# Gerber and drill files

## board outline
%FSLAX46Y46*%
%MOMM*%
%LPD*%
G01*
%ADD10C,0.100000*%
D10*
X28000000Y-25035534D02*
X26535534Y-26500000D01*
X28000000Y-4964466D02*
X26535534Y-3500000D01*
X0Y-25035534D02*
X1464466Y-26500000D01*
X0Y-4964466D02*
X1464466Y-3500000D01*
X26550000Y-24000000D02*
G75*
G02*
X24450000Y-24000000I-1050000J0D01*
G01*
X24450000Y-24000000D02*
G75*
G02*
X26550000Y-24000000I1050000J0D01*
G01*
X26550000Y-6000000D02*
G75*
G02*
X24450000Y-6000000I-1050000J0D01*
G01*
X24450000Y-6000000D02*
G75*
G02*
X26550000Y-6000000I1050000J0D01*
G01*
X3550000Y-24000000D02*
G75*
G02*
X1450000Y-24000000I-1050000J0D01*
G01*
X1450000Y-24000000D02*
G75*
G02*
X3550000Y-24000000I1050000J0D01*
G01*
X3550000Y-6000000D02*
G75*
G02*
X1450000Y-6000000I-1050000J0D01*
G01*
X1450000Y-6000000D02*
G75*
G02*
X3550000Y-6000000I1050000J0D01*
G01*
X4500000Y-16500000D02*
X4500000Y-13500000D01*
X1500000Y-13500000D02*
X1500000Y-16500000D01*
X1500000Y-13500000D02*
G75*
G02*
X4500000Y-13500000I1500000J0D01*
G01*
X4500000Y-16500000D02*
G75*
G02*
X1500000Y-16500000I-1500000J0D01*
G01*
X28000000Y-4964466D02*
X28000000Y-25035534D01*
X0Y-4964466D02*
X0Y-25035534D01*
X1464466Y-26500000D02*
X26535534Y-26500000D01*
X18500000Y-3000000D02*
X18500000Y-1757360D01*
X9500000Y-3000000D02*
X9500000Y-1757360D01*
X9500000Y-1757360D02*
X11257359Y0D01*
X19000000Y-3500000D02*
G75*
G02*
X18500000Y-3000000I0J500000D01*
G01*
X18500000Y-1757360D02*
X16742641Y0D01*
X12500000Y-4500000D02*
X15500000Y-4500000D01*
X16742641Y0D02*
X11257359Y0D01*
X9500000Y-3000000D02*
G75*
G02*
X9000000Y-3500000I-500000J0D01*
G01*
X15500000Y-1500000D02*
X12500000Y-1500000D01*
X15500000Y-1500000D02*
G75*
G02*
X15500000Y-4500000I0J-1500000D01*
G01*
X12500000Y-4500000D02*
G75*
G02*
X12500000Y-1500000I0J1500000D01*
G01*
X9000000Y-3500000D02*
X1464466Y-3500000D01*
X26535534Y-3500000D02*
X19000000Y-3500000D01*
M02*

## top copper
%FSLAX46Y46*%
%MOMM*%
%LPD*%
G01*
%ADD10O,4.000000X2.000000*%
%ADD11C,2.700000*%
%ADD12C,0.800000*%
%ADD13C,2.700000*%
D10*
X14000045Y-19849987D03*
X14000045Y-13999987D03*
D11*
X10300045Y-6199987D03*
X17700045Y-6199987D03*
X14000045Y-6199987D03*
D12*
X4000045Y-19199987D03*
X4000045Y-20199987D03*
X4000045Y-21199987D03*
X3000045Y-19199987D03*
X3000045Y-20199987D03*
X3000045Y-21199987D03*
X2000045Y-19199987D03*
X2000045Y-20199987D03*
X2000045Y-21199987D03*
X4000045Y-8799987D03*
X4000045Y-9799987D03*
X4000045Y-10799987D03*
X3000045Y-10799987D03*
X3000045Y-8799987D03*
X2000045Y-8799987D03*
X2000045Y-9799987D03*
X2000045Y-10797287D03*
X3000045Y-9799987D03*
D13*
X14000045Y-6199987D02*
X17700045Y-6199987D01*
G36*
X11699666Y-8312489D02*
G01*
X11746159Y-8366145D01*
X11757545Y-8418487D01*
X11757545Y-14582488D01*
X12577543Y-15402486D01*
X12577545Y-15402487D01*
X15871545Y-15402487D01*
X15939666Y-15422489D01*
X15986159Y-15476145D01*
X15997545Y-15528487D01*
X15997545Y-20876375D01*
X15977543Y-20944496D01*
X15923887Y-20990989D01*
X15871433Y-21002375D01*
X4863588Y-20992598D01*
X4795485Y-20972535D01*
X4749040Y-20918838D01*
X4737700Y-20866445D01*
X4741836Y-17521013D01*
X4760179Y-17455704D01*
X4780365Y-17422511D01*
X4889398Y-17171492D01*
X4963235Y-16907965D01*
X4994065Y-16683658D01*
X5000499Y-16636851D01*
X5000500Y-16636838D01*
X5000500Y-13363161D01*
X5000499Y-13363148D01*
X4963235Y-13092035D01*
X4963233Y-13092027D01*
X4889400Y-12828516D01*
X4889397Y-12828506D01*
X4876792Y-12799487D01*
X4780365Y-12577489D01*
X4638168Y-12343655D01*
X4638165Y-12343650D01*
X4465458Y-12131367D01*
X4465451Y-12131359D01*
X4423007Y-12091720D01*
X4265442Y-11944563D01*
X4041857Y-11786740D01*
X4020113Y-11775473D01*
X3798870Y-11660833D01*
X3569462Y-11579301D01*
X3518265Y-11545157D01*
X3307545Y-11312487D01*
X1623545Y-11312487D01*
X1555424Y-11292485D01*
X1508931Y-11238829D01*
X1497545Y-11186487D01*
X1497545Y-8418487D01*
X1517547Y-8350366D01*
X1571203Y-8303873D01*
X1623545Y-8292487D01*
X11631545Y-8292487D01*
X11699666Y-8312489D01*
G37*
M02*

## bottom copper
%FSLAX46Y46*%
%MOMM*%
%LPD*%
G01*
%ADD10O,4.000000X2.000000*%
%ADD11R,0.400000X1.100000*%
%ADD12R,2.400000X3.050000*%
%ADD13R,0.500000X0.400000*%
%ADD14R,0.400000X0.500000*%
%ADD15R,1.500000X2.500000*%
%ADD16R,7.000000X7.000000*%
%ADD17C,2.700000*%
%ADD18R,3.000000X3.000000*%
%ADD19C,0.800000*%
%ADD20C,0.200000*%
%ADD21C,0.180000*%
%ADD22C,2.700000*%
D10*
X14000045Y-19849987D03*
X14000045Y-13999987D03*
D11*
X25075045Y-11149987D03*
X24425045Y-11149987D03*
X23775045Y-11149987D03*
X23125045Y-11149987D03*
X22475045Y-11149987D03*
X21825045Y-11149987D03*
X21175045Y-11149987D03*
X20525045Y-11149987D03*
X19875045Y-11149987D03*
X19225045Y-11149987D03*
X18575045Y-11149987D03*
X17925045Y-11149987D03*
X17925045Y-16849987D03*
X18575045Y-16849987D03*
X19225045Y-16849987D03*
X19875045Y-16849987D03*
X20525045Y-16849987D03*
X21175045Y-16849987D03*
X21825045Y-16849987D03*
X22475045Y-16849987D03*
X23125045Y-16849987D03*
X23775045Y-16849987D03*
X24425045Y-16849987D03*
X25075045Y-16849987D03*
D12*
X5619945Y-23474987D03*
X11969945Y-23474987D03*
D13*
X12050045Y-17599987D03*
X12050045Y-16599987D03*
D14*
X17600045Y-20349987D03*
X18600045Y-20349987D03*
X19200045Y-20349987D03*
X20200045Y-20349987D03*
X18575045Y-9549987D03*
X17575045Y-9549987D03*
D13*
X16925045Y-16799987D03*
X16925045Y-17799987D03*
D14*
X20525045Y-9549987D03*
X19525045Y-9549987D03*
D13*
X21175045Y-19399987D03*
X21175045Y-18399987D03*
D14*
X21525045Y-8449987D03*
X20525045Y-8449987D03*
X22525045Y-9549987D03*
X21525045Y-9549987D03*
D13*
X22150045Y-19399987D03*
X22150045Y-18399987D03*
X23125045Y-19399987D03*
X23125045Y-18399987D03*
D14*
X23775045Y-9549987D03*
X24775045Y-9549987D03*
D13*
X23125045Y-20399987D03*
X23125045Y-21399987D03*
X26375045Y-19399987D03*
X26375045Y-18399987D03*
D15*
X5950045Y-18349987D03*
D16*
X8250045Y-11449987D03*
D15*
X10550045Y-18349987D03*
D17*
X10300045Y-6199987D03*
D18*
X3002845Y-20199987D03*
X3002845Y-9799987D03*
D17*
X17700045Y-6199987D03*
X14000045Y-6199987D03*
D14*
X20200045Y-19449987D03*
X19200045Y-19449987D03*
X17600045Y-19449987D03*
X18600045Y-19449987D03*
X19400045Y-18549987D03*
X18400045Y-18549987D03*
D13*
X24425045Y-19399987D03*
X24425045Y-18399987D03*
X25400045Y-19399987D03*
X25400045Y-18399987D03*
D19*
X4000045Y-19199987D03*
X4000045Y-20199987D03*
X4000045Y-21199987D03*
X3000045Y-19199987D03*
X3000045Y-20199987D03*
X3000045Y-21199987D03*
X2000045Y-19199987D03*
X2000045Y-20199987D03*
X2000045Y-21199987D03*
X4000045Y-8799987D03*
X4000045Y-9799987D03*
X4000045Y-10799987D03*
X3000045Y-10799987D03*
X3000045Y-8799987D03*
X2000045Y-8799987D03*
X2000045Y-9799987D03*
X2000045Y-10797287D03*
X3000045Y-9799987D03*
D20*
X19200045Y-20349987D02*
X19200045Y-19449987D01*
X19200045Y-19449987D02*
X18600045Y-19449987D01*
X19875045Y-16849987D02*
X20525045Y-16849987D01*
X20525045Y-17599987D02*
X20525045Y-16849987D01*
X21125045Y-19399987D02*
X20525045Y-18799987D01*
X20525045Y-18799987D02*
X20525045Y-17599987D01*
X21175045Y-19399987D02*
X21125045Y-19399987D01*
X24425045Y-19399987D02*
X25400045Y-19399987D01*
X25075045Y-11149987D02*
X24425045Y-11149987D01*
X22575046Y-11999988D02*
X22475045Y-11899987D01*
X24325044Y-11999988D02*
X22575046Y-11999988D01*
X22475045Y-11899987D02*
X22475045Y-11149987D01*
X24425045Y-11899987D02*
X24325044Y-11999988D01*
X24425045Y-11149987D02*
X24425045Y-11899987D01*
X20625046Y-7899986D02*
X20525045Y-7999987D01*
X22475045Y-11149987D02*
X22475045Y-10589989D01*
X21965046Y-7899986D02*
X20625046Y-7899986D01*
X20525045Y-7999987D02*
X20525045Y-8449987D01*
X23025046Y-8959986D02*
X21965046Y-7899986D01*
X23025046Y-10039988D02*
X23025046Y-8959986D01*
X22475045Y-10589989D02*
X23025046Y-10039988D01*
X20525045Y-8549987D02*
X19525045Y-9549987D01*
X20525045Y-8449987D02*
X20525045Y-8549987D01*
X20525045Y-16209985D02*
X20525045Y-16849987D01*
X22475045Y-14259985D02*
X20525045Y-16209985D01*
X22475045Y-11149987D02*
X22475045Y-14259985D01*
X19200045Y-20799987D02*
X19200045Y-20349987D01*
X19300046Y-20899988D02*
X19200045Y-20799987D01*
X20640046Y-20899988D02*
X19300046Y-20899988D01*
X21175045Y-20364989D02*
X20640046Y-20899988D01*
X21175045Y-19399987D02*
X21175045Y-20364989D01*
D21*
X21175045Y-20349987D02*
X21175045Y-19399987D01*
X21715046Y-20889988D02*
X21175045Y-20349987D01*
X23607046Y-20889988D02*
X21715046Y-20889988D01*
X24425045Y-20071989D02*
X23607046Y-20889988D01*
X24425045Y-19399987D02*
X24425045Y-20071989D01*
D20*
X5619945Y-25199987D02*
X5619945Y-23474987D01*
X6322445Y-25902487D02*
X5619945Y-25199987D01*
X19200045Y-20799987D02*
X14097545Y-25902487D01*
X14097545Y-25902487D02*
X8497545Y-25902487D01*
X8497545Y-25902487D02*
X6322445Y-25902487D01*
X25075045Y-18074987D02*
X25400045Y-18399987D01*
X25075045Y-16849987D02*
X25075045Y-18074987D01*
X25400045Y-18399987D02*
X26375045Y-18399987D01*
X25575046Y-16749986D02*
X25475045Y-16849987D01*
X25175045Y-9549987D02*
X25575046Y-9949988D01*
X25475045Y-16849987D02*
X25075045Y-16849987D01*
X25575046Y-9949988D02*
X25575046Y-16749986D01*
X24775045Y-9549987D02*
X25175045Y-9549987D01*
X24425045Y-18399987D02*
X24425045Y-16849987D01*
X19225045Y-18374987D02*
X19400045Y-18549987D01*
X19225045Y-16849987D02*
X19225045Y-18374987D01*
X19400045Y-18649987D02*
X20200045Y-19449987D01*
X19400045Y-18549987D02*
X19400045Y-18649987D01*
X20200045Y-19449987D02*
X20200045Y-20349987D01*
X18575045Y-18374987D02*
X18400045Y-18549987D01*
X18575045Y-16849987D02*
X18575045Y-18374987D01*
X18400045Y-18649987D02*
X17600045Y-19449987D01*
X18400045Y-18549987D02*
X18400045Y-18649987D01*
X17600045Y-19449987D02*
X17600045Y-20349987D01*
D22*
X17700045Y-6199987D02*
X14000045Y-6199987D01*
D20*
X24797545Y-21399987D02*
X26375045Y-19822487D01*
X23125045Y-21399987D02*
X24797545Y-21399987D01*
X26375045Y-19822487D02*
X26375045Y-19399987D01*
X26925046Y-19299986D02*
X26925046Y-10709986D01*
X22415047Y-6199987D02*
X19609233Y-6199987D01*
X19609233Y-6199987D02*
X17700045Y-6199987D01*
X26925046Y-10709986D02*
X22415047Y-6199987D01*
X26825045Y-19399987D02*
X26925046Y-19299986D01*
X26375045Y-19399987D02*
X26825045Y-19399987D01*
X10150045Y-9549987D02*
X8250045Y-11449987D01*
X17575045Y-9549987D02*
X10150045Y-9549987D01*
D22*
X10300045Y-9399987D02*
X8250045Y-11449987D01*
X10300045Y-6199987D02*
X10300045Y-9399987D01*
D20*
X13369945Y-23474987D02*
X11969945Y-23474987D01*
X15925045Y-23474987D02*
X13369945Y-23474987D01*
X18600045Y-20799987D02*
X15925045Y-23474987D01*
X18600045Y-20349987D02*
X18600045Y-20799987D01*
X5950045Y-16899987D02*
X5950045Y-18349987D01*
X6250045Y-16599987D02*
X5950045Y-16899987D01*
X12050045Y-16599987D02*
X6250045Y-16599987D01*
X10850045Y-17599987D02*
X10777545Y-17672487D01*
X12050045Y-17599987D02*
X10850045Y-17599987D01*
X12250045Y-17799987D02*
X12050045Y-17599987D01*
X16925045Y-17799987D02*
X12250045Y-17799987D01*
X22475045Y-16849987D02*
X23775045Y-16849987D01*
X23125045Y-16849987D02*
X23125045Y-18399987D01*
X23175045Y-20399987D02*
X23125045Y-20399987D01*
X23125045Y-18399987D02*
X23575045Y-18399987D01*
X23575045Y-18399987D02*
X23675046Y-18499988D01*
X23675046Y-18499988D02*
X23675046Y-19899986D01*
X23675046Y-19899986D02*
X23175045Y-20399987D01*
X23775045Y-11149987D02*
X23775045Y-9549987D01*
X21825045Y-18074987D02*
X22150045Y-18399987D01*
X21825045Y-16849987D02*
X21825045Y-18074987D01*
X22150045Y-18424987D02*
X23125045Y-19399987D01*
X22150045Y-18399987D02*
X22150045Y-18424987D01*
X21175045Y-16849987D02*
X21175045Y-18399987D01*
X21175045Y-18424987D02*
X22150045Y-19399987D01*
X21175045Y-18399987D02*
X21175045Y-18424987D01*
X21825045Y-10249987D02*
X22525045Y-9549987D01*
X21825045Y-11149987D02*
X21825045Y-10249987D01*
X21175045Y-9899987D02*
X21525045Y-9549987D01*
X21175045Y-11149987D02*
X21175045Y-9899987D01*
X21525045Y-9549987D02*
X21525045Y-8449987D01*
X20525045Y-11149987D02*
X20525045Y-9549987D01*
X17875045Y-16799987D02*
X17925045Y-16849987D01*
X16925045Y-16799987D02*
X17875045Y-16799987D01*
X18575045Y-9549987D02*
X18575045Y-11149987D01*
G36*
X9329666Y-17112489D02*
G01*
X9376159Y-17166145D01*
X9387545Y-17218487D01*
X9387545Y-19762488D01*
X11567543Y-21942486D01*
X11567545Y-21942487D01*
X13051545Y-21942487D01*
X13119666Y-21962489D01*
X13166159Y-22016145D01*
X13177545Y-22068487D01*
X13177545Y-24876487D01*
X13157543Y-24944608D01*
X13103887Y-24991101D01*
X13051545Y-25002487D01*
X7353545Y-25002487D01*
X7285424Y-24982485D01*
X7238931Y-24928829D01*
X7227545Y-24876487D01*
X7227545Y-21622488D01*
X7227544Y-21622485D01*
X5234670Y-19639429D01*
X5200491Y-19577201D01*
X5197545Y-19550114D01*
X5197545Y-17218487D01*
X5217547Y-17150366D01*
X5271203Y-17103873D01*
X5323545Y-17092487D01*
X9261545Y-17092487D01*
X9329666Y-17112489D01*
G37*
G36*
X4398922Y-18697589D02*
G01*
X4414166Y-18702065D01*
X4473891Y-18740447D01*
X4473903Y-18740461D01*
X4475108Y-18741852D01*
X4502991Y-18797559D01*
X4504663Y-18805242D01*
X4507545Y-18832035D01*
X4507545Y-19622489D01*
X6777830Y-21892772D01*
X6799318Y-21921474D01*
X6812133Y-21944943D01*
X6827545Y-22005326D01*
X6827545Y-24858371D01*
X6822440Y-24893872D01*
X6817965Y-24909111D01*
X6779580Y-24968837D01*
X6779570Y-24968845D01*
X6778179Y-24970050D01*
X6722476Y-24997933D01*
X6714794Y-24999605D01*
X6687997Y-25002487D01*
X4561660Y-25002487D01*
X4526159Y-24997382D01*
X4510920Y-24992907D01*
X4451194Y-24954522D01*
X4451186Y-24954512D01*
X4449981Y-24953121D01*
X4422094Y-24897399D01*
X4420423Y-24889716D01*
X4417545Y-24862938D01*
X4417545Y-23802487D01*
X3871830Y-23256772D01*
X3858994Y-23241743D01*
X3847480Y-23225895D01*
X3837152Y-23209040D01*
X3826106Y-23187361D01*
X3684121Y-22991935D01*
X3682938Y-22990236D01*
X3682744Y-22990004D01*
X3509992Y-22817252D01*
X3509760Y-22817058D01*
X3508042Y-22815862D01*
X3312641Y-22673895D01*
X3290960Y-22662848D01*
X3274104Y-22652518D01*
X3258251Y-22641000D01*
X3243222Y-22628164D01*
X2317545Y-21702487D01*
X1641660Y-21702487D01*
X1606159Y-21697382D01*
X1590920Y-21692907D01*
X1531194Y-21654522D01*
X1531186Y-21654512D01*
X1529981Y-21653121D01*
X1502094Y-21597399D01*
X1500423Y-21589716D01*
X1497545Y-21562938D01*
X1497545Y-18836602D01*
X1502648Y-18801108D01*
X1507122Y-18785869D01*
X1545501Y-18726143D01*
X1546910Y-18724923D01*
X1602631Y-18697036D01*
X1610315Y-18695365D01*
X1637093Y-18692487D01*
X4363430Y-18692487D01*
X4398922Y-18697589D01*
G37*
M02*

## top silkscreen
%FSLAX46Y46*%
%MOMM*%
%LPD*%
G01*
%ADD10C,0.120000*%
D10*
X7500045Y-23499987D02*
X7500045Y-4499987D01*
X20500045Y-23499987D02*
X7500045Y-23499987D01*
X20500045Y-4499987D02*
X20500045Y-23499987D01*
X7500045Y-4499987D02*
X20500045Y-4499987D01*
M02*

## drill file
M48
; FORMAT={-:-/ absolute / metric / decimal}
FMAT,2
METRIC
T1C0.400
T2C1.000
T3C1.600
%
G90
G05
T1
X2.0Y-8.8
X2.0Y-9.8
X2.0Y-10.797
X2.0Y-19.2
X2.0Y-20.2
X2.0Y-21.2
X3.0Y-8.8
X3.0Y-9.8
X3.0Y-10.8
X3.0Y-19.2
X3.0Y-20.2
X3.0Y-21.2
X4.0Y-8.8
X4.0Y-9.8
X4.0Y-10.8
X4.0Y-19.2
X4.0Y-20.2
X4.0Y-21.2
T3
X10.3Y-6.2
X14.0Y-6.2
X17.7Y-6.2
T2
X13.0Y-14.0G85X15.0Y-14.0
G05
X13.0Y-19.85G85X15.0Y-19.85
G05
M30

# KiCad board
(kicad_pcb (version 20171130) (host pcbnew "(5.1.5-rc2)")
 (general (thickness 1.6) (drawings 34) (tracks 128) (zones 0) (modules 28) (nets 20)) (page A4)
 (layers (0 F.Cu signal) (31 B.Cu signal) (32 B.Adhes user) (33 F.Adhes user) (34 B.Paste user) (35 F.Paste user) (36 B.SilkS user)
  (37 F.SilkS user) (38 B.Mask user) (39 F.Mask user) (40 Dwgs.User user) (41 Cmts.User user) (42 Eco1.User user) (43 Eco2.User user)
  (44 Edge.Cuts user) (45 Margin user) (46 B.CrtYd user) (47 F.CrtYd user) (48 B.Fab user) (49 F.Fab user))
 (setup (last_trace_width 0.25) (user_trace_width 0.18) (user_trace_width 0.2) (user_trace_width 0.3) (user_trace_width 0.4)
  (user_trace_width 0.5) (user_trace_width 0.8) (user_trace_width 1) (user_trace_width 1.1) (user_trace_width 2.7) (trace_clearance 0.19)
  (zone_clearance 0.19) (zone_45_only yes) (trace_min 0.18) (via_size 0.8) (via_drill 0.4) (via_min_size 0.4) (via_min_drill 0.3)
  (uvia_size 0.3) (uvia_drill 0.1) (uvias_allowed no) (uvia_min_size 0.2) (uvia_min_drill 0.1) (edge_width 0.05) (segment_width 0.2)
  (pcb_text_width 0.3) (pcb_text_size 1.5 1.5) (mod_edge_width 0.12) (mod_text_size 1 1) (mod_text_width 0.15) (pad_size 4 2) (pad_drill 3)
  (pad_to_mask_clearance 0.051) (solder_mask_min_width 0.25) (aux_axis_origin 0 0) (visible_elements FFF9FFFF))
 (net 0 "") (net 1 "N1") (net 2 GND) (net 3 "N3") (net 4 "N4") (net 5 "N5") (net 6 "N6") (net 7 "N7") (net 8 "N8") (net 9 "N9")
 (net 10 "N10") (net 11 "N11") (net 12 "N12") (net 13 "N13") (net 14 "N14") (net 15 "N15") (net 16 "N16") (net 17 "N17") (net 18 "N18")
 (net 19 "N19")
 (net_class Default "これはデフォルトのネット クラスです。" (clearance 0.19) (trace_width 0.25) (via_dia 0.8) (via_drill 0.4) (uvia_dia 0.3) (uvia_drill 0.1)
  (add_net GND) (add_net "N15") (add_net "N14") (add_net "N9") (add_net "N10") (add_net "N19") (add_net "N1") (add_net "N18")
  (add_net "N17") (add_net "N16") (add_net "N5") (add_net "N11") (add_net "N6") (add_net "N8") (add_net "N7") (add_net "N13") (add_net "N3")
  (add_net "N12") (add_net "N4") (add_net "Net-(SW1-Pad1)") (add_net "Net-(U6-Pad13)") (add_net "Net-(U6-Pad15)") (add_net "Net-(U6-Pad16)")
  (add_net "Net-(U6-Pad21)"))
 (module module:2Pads (layer F.Cu) (at 7.500045 4.499987)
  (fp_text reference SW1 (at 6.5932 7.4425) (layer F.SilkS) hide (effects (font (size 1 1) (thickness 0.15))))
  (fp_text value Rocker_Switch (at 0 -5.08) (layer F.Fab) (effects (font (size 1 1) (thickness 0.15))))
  (pad 2 thru_hole oval (at 6.5 15.35) (size 4 2) (drill oval 3 1) (layers *.Cu *.Mask) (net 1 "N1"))
  (pad 1 thru_hole oval (at 6.5 9.5) (size 4 2) (drill oval 3 1) (layers *.Cu *.Mask)))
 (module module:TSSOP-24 (layer B.Cu) (at 21.500045 13.999987 90)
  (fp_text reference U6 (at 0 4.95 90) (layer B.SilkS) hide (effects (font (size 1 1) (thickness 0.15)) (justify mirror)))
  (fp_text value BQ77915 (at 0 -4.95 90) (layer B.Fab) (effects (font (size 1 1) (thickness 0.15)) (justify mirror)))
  (pad 24 smd rect (at 2.85 3.575 90) (size 1.1 0.4) (layers B.Cu B.Paste B.Mask) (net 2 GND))
  (pad 23 smd rect (at 2.85 2.925 90) (size 1.1 0.4) (layers B.Cu B.Paste B.Mask) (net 2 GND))
  (pad 22 smd rect (at 2.85 2.275 90) (size 1.1 0.4) (layers B.Cu B.Paste B.Mask) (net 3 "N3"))
  (pad 21 smd rect (at 2.85 1.625 90) (size 1.1 0.4) (layers B.Cu B.Paste B.Mask))
  (pad 20 smd rect (at 2.85 0.975 90) (size 1.1 0.4) (layers B.Cu B.Paste B.Mask) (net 2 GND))
  (pad 19 smd rect (at 2.85 0.325 90) (size 1.1 0.4) (layers B.Cu B.Paste B.Mask) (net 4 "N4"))
  (pad 18 smd rect (at 2.85 -0.325 90) (size 1.1 0.4) (layers B.Cu B.Paste B.Mask) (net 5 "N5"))
  (pad 17 smd rect (at 2.85 -0.975 90) (size 1.1 0.4) (layers B.Cu B.Paste B.Mask) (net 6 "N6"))
  (pad 16 smd rect (at 2.85 -1.625 90) (size 1.1 0.4) (layers B.Cu B.Paste B.Mask))
  (pad 15 smd rect (at 2.85 -2.275 90) (size 1.1 0.4) (layers B.Cu B.Paste B.Mask))
  (pad 14 smd rect (at 2.85 -2.925 90) (size 1.1 0.4) (layers B.Cu B.Paste B.Mask) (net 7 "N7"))
  (pad 13 smd rect (at 2.85 -3.575 90) (size 1.1 0.4) (layers B.Cu B.Paste B.Mask))
  (pad 12 smd rect (at -2.85 -3.575 90) (size 1.1 0.4) (layers B.Cu B.Paste B.Mask) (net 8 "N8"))
  (pad 11 smd rect (at -2.85 -2.925 90) (size 1.1 0.4) (layers B.Cu B.Paste B.Mask) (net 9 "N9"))
  (pad 10 smd rect (at -2.85 -2.275 90) (size 1.1 0.4) (layers B.Cu B.Paste B.Mask) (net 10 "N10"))
  (pad 9 smd rect (at -2.85 -1.625 90) (size 1.1 0.4) (layers B.Cu B.Paste B.Mask) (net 2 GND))
  (pad 8 smd rect (at -2.85 -0.975 90) (size 1.1 0.4) (layers B.Cu B.Paste B.Mask) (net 2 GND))
  (pad 7 smd rect (at -2.85 -0.325 90) (size 1.1 0.4) (layers B.Cu B.Paste B.Mask) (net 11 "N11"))
  (pad 6 smd rect (at -2.85 0.325 90) (size 1.1 0.4) (layers B.Cu B.Paste B.Mask) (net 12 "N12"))
  (pad 5 smd rect (at -2.85 0.975 90) (size 1.1 0.4) (layers B.Cu B.Paste B.Mask) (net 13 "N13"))
  (pad 4 smd rect (at -2.85 1.625 90) (size 1.1 0.4) (layers B.Cu B.Paste B.Mask) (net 13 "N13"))
  (pad 3 smd rect (at -2.85 2.275 90) (size 1.1 0.4) (layers B.Cu B.Paste B.Mask) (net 13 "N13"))
  (pad 2 smd rect (at -2.85 2.925 90) (size 1.1 0.4) (layers B.Cu B.Paste B.Mask) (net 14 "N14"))
  (pad 1 smd rect (at -2.85 3.575 90) (size 1.1 0.4) (layers B.Cu B.Paste B.Mask) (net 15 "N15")))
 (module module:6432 (layer B.Cu) (at 8.794945 23.474987 180)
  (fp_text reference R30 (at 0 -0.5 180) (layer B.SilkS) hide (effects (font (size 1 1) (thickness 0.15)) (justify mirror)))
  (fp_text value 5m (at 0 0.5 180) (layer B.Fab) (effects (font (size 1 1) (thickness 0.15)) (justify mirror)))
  (pad 2 smd rect (at 3.175 0 180) (size 2.4 3.05) (layers B.Cu B.Paste B.Mask) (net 2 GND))
  (pad 1 smd rect (at -3.175 0 180) (size 2.4 3.05) (layers B.Cu B.Paste B.Mask) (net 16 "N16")))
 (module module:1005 (layer B.Cu) (at 12.050045 17.099987 270)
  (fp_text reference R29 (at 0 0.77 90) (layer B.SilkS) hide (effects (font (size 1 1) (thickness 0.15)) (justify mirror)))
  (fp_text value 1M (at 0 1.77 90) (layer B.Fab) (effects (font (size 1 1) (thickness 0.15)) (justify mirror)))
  (pad 2 smd rect (at 0.5 0 270) (size 0.4 0.5) (layers B.Cu B.Paste B.Mask) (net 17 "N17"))
  (pad 1 smd rect (at -0.5 0 270) (size 0.4 0.5) (layers B.Cu B.Paste B.Mask) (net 16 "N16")))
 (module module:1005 (layer B.Cu) (at 18.100045 20.349987 180)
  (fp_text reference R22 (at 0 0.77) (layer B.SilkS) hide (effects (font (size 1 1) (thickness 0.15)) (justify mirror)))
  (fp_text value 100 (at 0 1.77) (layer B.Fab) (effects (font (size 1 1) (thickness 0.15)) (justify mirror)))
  (pad 2 smd rect (at 0.5 0 180) (size 0.4 0.5) (layers B.Cu B.Paste B.Mask) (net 9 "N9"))
  (pad 1 smd rect (at -0.5 0 180) (size 0.4 0.5) (layers B.Cu B.Paste B.Mask) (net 16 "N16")))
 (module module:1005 (layer B.Cu) (at 19.700045 20.349987 180)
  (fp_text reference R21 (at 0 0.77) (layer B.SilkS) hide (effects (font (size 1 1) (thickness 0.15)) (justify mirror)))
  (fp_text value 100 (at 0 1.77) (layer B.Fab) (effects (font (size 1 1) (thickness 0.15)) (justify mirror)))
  (pad 2 smd rect (at 0.5 0 180) (size 0.4 0.5) (layers B.Cu B.Paste B.Mask) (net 2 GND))
  (pad 1 smd rect (at -0.5 0 180) (size 0.4 0.5) (layers B.Cu B.Paste B.Mask) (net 10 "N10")))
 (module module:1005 (layer B.Cu) (at 18.075045 9.549987)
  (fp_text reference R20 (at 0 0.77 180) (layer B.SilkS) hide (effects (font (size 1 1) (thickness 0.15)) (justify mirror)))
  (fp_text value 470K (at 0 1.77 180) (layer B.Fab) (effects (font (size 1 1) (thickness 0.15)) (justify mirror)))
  (pad 2 smd rect (at 0.5 0) (size 0.4 0.5) (layers B.Cu B.Paste B.Mask) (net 7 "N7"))
  (pad 1 smd rect (at -0.5 0) (size 0.4 0.5) (layers B.Cu B.Paste B.Mask) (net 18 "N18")))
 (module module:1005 (layer B.Cu) (at 16.925045 17.299987 90)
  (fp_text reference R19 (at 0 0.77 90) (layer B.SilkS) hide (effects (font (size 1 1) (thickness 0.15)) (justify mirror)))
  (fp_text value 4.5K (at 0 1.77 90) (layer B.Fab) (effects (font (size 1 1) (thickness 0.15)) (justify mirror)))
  (pad 2 smd rect (at 0.5 0 90) (size 0.4 0.5) (layers B.Cu B.Paste B.Mask) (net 8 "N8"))
  (pad 1 smd rect (at -0.5 0 90) (size 0.4 0.5) (layers B.Cu B.Paste B.Mask) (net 17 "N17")))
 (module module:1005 (layer B.Cu) (at 20.025045 9.549987)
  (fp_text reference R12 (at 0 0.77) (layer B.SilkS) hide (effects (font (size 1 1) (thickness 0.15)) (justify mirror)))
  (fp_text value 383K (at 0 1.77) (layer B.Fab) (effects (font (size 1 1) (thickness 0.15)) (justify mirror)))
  (pad 2 smd rect (at 0.5 0) (size 0.4 0.5) (layers B.Cu B.Paste B.Mask) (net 6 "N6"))
  (pad 1 smd rect (at -0.5 0) (size 0.4 0.5) (layers B.Cu B.Paste B.Mask) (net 2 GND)))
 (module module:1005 (layer B.Cu) (at 21.175045 18.899987 270)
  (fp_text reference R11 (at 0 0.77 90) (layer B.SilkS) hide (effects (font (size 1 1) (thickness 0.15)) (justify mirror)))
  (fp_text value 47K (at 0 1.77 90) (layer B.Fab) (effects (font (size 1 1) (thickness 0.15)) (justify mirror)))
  (pad 2 smd rect (at 0.5 0 270) (size 0.4 0.5) (layers B.Cu B.Paste B.Mask) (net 2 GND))
  (pad 1 smd rect (at -0.5 0 270) (size 0.4 0.5) (layers B.Cu B.Paste B.Mask) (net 11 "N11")))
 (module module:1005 (layer B.Cu) (at 21.025045 8.449987)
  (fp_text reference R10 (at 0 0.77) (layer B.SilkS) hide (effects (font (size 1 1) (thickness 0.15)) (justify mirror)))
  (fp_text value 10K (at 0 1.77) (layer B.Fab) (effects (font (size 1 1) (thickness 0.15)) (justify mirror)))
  (pad 2 smd rect (at 0.5 0) (size 0.4 0.5) (layers B.Cu B.Paste B.Mask) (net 5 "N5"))
  (pad 1 smd rect (at -0.5 0) (size 0.4 0.5) (layers B.Cu B.Paste B.Mask) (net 2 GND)))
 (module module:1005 (layer B.Cu) (at 22.025045 9.549987)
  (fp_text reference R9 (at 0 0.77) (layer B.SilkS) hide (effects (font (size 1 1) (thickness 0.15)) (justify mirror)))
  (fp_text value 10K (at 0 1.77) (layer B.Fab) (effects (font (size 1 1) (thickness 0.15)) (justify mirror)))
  (pad 2 smd rect (at 0.5 0) (size 0.4 0.5) (layers B.Cu B.Paste B.Mask) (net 4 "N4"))
  (pad 1 smd rect (at -0.5 0) (size 0.4 0.5) (layers B.Cu B.Paste B.Mask) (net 5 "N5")))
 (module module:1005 (layer B.Cu) (at 22.150045 18.899987 270)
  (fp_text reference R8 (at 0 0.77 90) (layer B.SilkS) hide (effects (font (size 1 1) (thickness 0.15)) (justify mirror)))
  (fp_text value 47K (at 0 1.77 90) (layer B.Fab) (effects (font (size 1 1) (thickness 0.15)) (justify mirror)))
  (pad 2 smd rect (at 0.5 0 270) (size 0.4 0.5) (layers B.Cu B.Paste B.Mask) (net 11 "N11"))
  (pad 1 smd rect (at -0.5 0 270) (size 0.4 0.5) (layers B.Cu B.Paste B.Mask) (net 12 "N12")))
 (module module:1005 (layer B.Cu) (at 23.125045 18.899987 270)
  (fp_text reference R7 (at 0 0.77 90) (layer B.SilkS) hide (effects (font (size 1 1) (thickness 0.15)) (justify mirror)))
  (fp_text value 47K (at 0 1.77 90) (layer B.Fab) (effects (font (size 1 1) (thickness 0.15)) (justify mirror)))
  (pad 2 smd rect (at 0.5 0 270) (size 0.4 0.5) (layers B.Cu B.Paste B.Mask) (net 12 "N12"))
  (pad 1 smd rect (at -0.5 0 270) (size 0.4 0.5) (layers B.Cu B.Paste B.Mask) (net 13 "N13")))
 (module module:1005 (layer B.Cu) (at 24.275045 9.549987 180)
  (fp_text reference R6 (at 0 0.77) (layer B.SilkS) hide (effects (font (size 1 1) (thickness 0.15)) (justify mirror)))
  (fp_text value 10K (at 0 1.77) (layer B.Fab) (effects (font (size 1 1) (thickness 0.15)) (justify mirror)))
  (pad 2 smd rect (at 0.5 0 180) (size 0.4 0.5) (layers B.Cu B.Paste B.Mask) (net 3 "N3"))
  (pad 1 smd rect (at -0.5 0 180) (size 0.4 0.5) (layers B.Cu B.Paste B.Mask) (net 15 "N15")))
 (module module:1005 (layer B.Cu) (at 23.125045 20.899987 90)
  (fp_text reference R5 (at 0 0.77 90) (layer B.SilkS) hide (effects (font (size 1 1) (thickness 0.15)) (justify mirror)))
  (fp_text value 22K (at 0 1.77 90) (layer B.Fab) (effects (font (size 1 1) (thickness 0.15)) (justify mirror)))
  (pad 2 smd rect (at 0.5 0 90) (size 0.4 0.5) (layers B.Cu B.Paste B.Mask) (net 13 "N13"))
  (pad 1 smd rect (at -0.5 0 90) (size 0.4 0.5) (layers B.Cu B.Paste B.Mask) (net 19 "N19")))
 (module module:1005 (layer B.Cu) (at 26.375045 18.899987 270)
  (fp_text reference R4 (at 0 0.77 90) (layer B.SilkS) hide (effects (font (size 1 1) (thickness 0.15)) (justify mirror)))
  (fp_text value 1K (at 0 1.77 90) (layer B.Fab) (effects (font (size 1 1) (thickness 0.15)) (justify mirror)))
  (pad 2 smd rect (at 0.5 0 270) (size 0.4 0.5) (layers B.Cu B.Paste B.Mask) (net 19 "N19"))
  (pad 1 smd rect (at -0.5 0 270) (size 0.4 0.5) (layers B.Cu B.Paste B.Mask) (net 15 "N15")))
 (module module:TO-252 (layer B.Cu) (at 8.250045 11.449987 180)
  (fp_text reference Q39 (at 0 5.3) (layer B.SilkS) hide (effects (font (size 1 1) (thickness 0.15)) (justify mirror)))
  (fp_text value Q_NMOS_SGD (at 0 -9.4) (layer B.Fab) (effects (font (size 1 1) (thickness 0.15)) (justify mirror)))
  (pad 3 smd rect (at 2.3 -6.9 180) (size 1.5 2.5) (layers B.Cu B.Paste B.Mask) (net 16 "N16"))
  (pad 2 smd rect (at 0 0 180) (size 7 7) (layers B.Cu B.Paste B.Mask) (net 18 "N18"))
  (pad 1 smd rect (at -2.3 -6.9 180) (size 1.5 2.5) (layers B.Cu B.Paste B.Mask) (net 17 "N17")))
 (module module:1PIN (layer F.Cu) (at 11.927545 5.782487 90)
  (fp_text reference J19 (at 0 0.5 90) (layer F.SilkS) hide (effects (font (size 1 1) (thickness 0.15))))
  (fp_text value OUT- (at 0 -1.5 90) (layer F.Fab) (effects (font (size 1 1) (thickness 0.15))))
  (pad 1 thru_hole circle (at -0.4175 -1.6275 90) (size 2.7 2.7) (drill 1.6) (layers *.Cu *.Mask) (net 18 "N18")))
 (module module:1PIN (layer B.Cu) (at 2.907545 20.342487 90)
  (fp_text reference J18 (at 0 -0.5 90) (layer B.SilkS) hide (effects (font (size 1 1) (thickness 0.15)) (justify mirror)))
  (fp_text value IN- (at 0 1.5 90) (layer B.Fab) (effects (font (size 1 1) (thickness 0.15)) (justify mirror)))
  (pad 1 smd rect (at 0.1425 0.0953 90) (size 3 3) (layers B.Cu B.Paste B.Mask) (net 2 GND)))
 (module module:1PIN (layer B.Cu) (at 2.997545 9.982487 90)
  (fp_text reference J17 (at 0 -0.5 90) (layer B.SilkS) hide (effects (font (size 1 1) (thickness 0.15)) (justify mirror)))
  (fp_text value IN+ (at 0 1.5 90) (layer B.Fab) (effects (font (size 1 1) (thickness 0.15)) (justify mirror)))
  (pad 1 smd rect (at 0.1825 0.0053 90) (size 3 3) (layers B.Cu B.Paste B.Mask) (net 1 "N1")))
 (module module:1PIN (layer F.Cu) (at 16.587545 5.832487 90)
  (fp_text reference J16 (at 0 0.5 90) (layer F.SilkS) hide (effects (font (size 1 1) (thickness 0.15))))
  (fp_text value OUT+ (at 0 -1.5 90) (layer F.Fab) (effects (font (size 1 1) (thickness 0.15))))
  (pad 1 thru_hole circle (at -0.3675 1.1125 90) (size 2.7 2.7) (drill 1.6) (layers *.Cu *.Mask) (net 19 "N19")))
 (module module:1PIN (layer F.Cu) (at 14.217545 5.792487 90)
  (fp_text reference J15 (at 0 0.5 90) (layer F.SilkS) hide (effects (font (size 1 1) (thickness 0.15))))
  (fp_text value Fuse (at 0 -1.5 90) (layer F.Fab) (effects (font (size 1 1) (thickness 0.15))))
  (pad 1 thru_hole circle (at -0.4075 -0.2175 90) (size 2.7 2.7) (drill 1.6) (layers *.Cu *.Mask) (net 19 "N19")))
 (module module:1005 (layer B.Cu) (at 19.700045 19.449987)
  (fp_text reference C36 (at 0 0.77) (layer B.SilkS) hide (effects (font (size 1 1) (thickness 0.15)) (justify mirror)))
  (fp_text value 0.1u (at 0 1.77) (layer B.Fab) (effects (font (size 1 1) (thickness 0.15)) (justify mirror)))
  (pad 2 smd rect (at 0.5 0) (size 0.4 0.5) (layers B.Cu B.Paste B.Mask) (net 10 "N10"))
  (pad 1 smd rect (at -0.5 0) (size 0.4 0.5) (layers B.Cu B.Paste B.Mask) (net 2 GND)))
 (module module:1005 (layer B.Cu) (at 18.100045 19.449987 180)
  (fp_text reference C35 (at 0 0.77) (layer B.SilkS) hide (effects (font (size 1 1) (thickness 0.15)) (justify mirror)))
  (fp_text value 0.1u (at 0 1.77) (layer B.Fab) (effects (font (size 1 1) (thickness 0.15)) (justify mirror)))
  (pad 2 smd rect (at 0.5 0 180) (size 0.4 0.5) (layers B.Cu B.Paste B.Mask) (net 9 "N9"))
  (pad 1 smd rect (at -0.5 0 180) (size 0.4 0.5) (layers B.Cu B.Paste B.Mask) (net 2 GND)))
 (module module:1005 (layer B.Cu) (at 18.900045 18.549987)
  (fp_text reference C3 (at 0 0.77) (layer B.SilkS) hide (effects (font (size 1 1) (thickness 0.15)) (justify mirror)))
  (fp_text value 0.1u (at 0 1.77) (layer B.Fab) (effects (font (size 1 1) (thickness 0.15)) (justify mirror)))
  (pad 2 smd rect (at 0.5 0) (size 0.4 0.5) (layers B.Cu B.Paste B.Mask) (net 10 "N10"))
  (pad 1 smd rect (at -0.5 0) (size 0.4 0.5) (layers B.Cu B.Paste B.Mask) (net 9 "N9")))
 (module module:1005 (layer B.Cu) (at 24.425045 18.899987 270)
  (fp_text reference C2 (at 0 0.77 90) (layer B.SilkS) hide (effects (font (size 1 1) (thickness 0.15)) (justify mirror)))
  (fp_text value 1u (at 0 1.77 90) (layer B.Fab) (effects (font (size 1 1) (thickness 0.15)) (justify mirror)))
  (pad 2 smd rect (at 0.5 0 270) (size 0.4 0.5) (layers B.Cu B.Paste B.Mask) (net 2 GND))
  (pad 1 smd rect (at -0.5 0 270) (size 0.4 0.5) (layers B.Cu B.Paste B.Mask) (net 14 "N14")))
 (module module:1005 (layer B.Cu) (at 25.400045 18.899987 270)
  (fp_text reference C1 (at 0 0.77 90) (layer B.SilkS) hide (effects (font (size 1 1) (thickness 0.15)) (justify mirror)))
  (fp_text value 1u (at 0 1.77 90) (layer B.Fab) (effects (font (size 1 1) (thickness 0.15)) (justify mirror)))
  (pad 2 smd rect (at 0.5 0 270) (size 0.4 0.5) (layers B.Cu B.Paste B.Mask) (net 2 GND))
  (pad 1 smd rect (at -0.5 0 270) (size 0.4 0.5) (layers B.Cu B.Paste B.Mask) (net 15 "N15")))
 (gr_line (start 7.500045 23.499987) (end 7.500045 4.499987) (layer F.SilkS) (width 0.12))
 (gr_line (start 20.500045 23.499987) (end 7.500045 23.499987) (layer F.SilkS) (width 0.12))
 (gr_line (start 20.500045 4.499987) (end 20.500045 23.499987) (layer F.SilkS) (width 0.12))
 (gr_line (start 7.500045 4.499987) (end 20.500045 4.499987) (layer F.SilkS) (width 0.12))
 (gr_line (start 28 25.035534) (end 26.535534 26.5) (layer Edge.Cuts) (width 0.1))
 (gr_line (start 28 4.964466) (end 26.535534 3.5) (layer Edge.Cuts) (width 0.1))
 (gr_line (start 0 25.035534) (end 1.464466 26.5) (layer Edge.Cuts) (width 0.1))
 (gr_line (start 0 4.964466) (end 1.464466 3.5) (layer Edge.Cuts) (width 0.1))
 (gr_circle (center 25.5 24) (end 25.5 22.95) (layer Edge.Cuts) (width 0.1))
 (gr_circle (center 25.5 6) (end 25.5 4.95) (layer Edge.Cuts) (width 0.1))
 (gr_circle (center 2.5 24) (end 2.5 22.95) (layer Edge.Cuts) (width 0.1))
 (gr_circle (center 2.5 6) (end 2.5 4.95) (layer Edge.Cuts) (width 0.1))
 (gr_line (start 4.5 16.5) (end 4.5 13.5) (layer Edge.Cuts) (width 0.1))
 (gr_line (start 1.5 13.5) (end 1.5 16.5) (layer Edge.Cuts) (width 0.1))
 (gr_arc (start 3 13.5) (end 4.5 13.5) (angle -180) (layer Edge.Cuts) (width 0.1))
 (gr_arc (start 3 16.5) (end 1.5 16.5) (angle -180) (layer Edge.Cuts) (width 0.1))
 (gr_line (start 28 4.964466) (end 28 25.035534) (layer Edge.Cuts) (width 0.1))
 (gr_line (start 0 4.964466) (end 0 25.035534) (layer Edge.Cuts) (width 0.1))
 (gr_line (start 1.464466 26.5) (end 26.535534 26.5) (layer Edge.Cuts) (width 0.1))
 (gr_line (start 18.5 3) (end 18.5 1.75736) (layer Edge.Cuts) (width 0.1))
 (gr_line (start 9.5 3) (end 9.5 1.75736) (layer Edge.Cuts) (width 0.1))
 (gr_line (start 9.5 1.75736) (end 11.257359 0) (layer Edge.Cuts) (width 0.1))
 (gr_arc (start 19 3) (end 18.5 3) (angle -90) (layer Edge.Cuts) (width 0.1))
 (gr_line (start 18.5 1.75736) (end 16.742641 0) (layer Edge.Cuts) (width 0.1))
 (gr_line (start 12.5 4.5) (end 15.5 4.5) (layer Edge.Cuts) (width 0.1))
 (gr_line (start 16.742641 0) (end 11.257359 0) (layer Edge.Cuts) (width 0.1))
 (gr_arc (start 9 3) (end 9 3.5) (angle -90) (layer Edge.Cuts) (width 0.1))
 (gr_line (start 15.5 1.5) (end 12.5 1.5) (layer Edge.Cuts) (width 0.1))
 (gr_arc (start 15.5 3) (end 15.5 4.5) (angle -180) (layer Edge.Cuts) (width 0.1))
 (gr_arc (start 12.5 3) (end 12.5 1.5) (angle -180) (layer Edge.Cuts) (width 0.1))
 (gr_line (start 9 3.5) (end 1.464466 3.5) (layer Edge.Cuts) (width 0.1))
 (gr_line (start 26.535534 3.5) (end 19 3.5) (layer Edge.Cuts) (width 0.1))
 (via (at 4.000045 19.199987) (size 0.8) (drill 0.4) (layers F.Cu B.Cu) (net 2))
 (via (at 4.000045 20.199987) (size 0.8) (drill 0.4) (layers F.Cu B.Cu) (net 2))
 (via (at 4.000045 21.199987) (size 0.8) (drill 0.4) (layers F.Cu B.Cu) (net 2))
 (via (at 3.000045 19.199987) (size 0.8) (drill 0.4) (layers F.Cu B.Cu) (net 2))
 (via (at 3.000045 20.199987) (size 0.8) (drill 0.4) (layers F.Cu B.Cu) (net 2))
 (via (at 3.000045 21.199987) (size 0.8) (drill 0.4) (layers F.Cu B.Cu) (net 2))
 (via (at 2.000045 19.199987) (size 0.8) (drill 0.4) (layers F.Cu B.Cu) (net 2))
 (via (at 2.000045 20.199987) (size 0.8) (drill 0.4) (layers F.Cu B.Cu) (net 2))
 (via (at 2.000045 21.199987) (size 0.8) (drill 0.4) (layers F.Cu B.Cu) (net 2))
 (segment (start 19.200045 20.349987) (end 19.200045 19.449987) (width 0.2) (layer B.Cu) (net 2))
 (segment (start 19.200045 19.449987) (end 18.600045 19.449987) (width 0.2) (layer B.Cu) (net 2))
 (segment (start 19.875045 16.849987) (end 20.525045 16.849987) (width 0.2) (layer B.Cu) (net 2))
 (segment (start 20.525045 17.599987) (end 20.525045 16.849987) (width 0.2) (layer B.Cu) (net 2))
 (segment (start 21.125045 19.399987) (end 20.525045 18.799987) (width 0.2) (layer B.Cu) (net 2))
 (segment (start 20.525045 18.799987) (end 20.525045 17.599987) (width 0.2) (layer B.Cu) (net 2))
 (segment (start 21.175045 19.399987) (end 21.125045 19.399987) (width 0.2) (layer B.Cu) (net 2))
 (segment (start 24.425045 19.399987) (end 25.400045 19.399987) (width 0.2) (layer B.Cu) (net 2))
 (segment (start 25.075045 11.149987) (end 24.425045 11.149987) (width 0.2) (layer B.Cu) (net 2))
 (segment (start 22.575046 11.999988) (end 22.475045 11.899987) (width 0.2) (layer B.Cu) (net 2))
 (segment (start 24.325044 11.999988) (end 22.575046 11.999988) (width 0.2) (layer B.Cu) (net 2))
 (segment (start 22.475045 11.899987) (end 22.475045 11.149987) (width 0.2) (layer B.Cu) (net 2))
 (segment (start 24.425045 11.899987) (end 24.325044 11.999988) (width 0.2) (layer B.Cu) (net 2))
 (segment (start 24.425045 11.149987) (end 24.425045 11.899987) (width 0.2) (layer B.Cu) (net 2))
 (segment (start 20.625046 7.899986) (end 20.525045 7.999987) (width 0.2) (layer B.Cu) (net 2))
 (segment (start 22.475045 11.149987) (end 22.475045 10.589989) (width 0.2) (layer B.Cu) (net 2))
 (segment (start 21.965046 7.899986) (end 20.625046 7.899986) (width 0.2) (layer B.Cu) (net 2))
 (segment (start 20.525045 7.999987) (end 20.525045 8.449987) (width 0.2) (layer B.Cu) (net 2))
 (segment (start 23.025046 8.959986) (end 21.965046 7.899986) (width 0.2) (layer B.Cu) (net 2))
 (segment (start 23.025046 10.039988) (end 23.025046 8.959986) (width 0.2) (layer B.Cu) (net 2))
 (segment (start 22.475045 10.589989) (end 23.025046 10.039988) (width 0.2) (layer B.Cu) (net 2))
 (segment (start 20.525045 8.549987) (end 19.525045 9.549987) (width 0.2) (layer B.Cu) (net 2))
 (segment (start 20.525045 8.449987) (end 20.525045 8.549987) (width 0.2) (layer B.Cu) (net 2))
 (segment (start 20.525045 16.209985) (end 20.525045 16.849987) (width 0.2) (layer B.Cu) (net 2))
 (segment (start 22.475045 14.259985) (end 20.525045 16.209985) (width 0.2) (layer B.Cu) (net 2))
 (segment (start 22.475045 11.149987) (end 22.475045 14.259985) (width 0.2) (layer B.Cu) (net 2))
 (segment (start 19.200045 20.799987) (end 19.200045 20.349987) (width 0.2) (layer B.Cu) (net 2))
 (segment (start 19.300046 20.899988) (end 19.200045 20.799987) (width 0.2) (layer B.Cu) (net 2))
 (segment (start 20.640046 20.899988) (end 19.300046 20.899988) (width 0.2) (layer B.Cu) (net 2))
 (segment (start 21.175045 20.364989) (end 20.640046 20.899988) (width 0.2) (layer B.Cu) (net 2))
 (segment (start 21.175045 19.399987) (end 21.175045 20.364989) (width 0.2) (layer B.Cu) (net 2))
 (segment (start 21.175045 20.349987) (end 21.175045 19.399987) (width 0.18) (layer B.Cu) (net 2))
 (segment (start 21.715046 20.889988) (end 21.175045 20.349987) (width 0.18) (layer B.Cu) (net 2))
 (segment (start 23.607046 20.889988) (end 21.715046 20.889988) (width 0.18) (layer B.Cu) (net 2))
 (segment (start 24.425045 20.071989) (end 23.607046 20.889988) (width 0.18) (layer B.Cu) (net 2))
 (segment (start 24.425045 19.399987) (end 24.425045 20.071989) (width 0.18) (layer B.Cu) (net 2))
 (segment (start 5.619945 25.199987) (end 5.619945 23.474987) (width 0.2) (layer B.Cu) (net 2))
 (segment (start 6.322445 25.902487) (end 5.619945 25.199987) (width 0.2) (layer B.Cu) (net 2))
 (segment (start 19.200045 20.799987) (end 14.097545 25.902487) (width 0.2) (layer B.Cu) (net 2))
 (segment (start 14.097545 25.902487) (end 8.497545 25.902487) (width 0.2) (layer B.Cu) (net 2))
 (segment (start 8.497545 25.902487) (end 6.322445 25.902487) (width 0.2) (layer B.Cu) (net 2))
 (segment (start 25.075045 18.074987) (end 25.400045 18.399987) (width 0.2) (layer B.Cu) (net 15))
 (segment (start 25.075045 16.849987) (end 25.075045 18.074987) (width 0.2) (layer B.Cu) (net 15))
 (segment (start 25.400045 18.399987) (end 26.375045 18.399987) (width 0.2) (layer B.Cu) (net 15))
 (segment (start 25.575046 16.749986) (end 25.475045 16.849987) (width 0.2) (layer B.Cu) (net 15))
 (segment (start 25.175045 9.549987) (end 25.575046 9.949988) (width 0.2) (layer B.Cu) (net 15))
 (segment (start 25.475045 16.849987) (end 25.075045 16.849987) (width 0.2) (layer B.Cu) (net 15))
 (segment (start 25.575046 9.949988) (end 25.575046 16.749986) (width 0.2) (layer B.Cu) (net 15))
 (segment (start 24.775045 9.549987) (end 25.175045 9.549987) (width 0.2) (layer B.Cu) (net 15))
 (segment (start 24.425045 18.399987) (end 24.425045 16.849987) (width 0.2) (layer B.Cu) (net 14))
 (segment (start 19.225045 18.374987) (end 19.400045 18.549987) (width 0.2) (layer B.Cu) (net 10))
 (segment (start 19.225045 16.849987) (end 19.225045 18.374987) (width 0.2) (layer B.Cu) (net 10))
 (segment (start 19.400045 18.649987) (end 20.200045 19.449987) (width 0.2) (layer B.Cu) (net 10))
 (segment (start 19.400045 18.549987) (end 19.400045 18.649987) (width 0.2) (layer B.Cu) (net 10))
 (segment (start 20.200045 19.449987) (end 20.200045 20.349987) (width 0.2) (layer B.Cu) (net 10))
 (segment (start 18.575045 18.374987) (end 18.400045 18.549987) (width 0.2) (layer B.Cu) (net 9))
 (segment (start 18.575045 16.849987) (end 18.575045 18.374987) (width 0.2) (layer B.Cu) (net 9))
 (segment (start 18.400045 18.649987) (end 17.600045 19.449987) (width 0.2) (layer B.Cu) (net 9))
 (segment (start 18.400045 18.549987) (end 18.400045 18.649987) (width 0.2) (layer B.Cu) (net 9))
 (segment (start 17.600045 19.449987) (end 17.600045 20.349987) (width 0.2) (layer B.Cu) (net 9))
 (segment (start 14.000045 6.199987) (end 17.700045 6.199987) (width 2.7) (layer F.Cu) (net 19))
 (segment (start 17.700045 6.199987) (end 14.000045 6.199987) (width 2.7) (layer B.Cu) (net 19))
 (segment (start 24.797545 21.399987) (end 26.375045 19.822487) (width 0.2) (layer B.Cu) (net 19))
 (segment (start 23.125045 21.399987) (end 24.797545 21.399987) (width 0.2) (layer B.Cu) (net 19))
 (segment (start 26.375045 19.822487) (end 26.375045 19.399987) (width 0.2) (layer B.Cu) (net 19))
 (segment (start 26.925046 19.299986) (end 26.925046 10.709986) (width 0.2) (layer B.Cu) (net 19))
 (segment (start 22.415047 6.199987) (end 19.609233 6.199987) (width 0.2) (layer B.Cu) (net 19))
 (segment (start 19.609233 6.199987) (end 17.700045 6.199987) (width 0.2) (layer B.Cu) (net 19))
 (segment (start 26.925046 10.709986) (end 22.415047 6.199987) (width 0.2) (layer B.Cu) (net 19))
 (segment (start 26.825045 19.399987) (end 26.925046 19.299986) (width 0.2) (layer B.Cu) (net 19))
 (segment (start 26.375045 19.399987) (end 26.825045 19.399987) (width 0.2) (layer B.Cu) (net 19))
 (via (at 4.000045 8.799987) (size 0.8) (drill 0.4) (layers F.Cu B.Cu) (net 1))
 (via (at 4.000045 9.799987) (size 0.8) (drill 0.4) (layers F.Cu B.Cu) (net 1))
 (via (at 4.000045 10.799987) (size 0.8) (drill 0.4) (layers F.Cu B.Cu) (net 1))
 (via (at 3.000045 10.799987) (size 0.8) (drill 0.4) (layers F.Cu B.Cu) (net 1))
 (via (at 3.000045 8.799987) (size 0.8) (drill 0.4) (layers F.Cu B.Cu) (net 1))
 (via (at 2.000045 8.799987) (size 0.8) (drill 0.4) (layers F.Cu B.Cu) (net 1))
 (via (at 2.000045 9.799987) (size 0.8) (drill 0.4) (layers F.Cu B.Cu) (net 1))
 (via (at 2.000045 10.797287) (size 0.8) (drill 0.4) (layers F.Cu B.Cu) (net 1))
 (via (at 3.000045 9.799987) (size 0.8) (drill 0.4) (layers F.Cu B.Cu) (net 1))
 (segment (start 10.150045 9.549987) (end 8.250045 11.449987) (width 0.2) (layer B.Cu) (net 18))
 (segment (start 17.575045 9.549987) (end 10.150045 9.549987) (width 0.2) (layer B.Cu) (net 18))
 (segment (start 10.300045 9.399987) (end 8.250045 11.449987) (width 2.7) (layer B.Cu) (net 18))
 (segment (start 10.300045 6.199987) (end 10.300045 9.399987) (width 2.7) (layer B.Cu) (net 18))
 (segment (start 13.369945 23.474987) (end 11.969945 23.474987) (width 0.2) (layer B.Cu) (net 16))
 (segment (start 15.925045 23.474987) (end 13.369945 23.474987) (width 0.2) (layer B.Cu) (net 16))
 (segment (start 18.600045 20.799987) (end 15.925045 23.474987) (width 0.2) (layer B.Cu) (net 16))
 (segment (start 18.600045 20.349987) (end 18.600045 20.799987) (width 0.2) (layer B.Cu) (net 16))
 (segment (start 5.950045 16.899987) (end 5.950045 18.349987) (width 0.2) (layer B.Cu) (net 16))
 (segment (start 6.250045 16.599987) (end 5.950045 16.899987) (width 0.2) (layer B.Cu) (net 16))
 (segment (start 12.050045 16.599987) (end 6.250045 16.599987) (width 0.2) (layer B.Cu) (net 16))
 (segment (start 10.850045 17.599987) (end 10.777545 17.672487) (width 0.2) (layer B.Cu) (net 17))
 (segment (start 12.050045 17.599987) (end 10.850045 17.599987) (width 0.2) (layer B.Cu) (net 17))
 (segment (start 12.250045 17.799987) (end 12.050045 17.599987) (width 0.2) (layer B.Cu) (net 17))
 (segment (start 16.925045 17.799987) (end 12.250045 17.799987) (width 0.2) (layer B.Cu) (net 17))
 (segment (start 22.475045 16.849987) (end 23.775045 16.849987) (width 0.2) (layer B.Cu) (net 13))
 (segment (start 23.125045 16.849987) (end 23.125045 18.399987) (width 0.2) (layer B.Cu) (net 13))
 (segment (start 23.175045 20.399987) (end 23.125045 20.399987) (width 0.2) (layer B.Cu) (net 13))
 (segment (start 23.125045 18.399987) (end 23.575045 18.399987) (width 0.2) (layer B.Cu) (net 13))
 (segment (start 23.575045 18.399987) (end 23.675046 18.499988) (width 0.2) (layer B.Cu) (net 13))
 (segment (start 23.675046 18.499988) (end 23.675046 19.899986) (width 0.2) (layer B.Cu) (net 13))
 (segment (start 23.675046 19.899986) (end 23.175045 20.399987) (width 0.2) (layer B.Cu) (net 13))
 (segment (start 23.775045 11.149987) (end 23.775045 9.549987) (width 0.2) (layer B.Cu) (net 3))
 (segment (start 21.825045 18.074987) (end 22.150045 18.399987) (width 0.2) (layer B.Cu) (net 12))
 (segment (start 21.825045 16.849987) (end 21.825045 18.074987) (width 0.2) (layer B.Cu) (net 12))
 (segment (start 22.150045 18.424987) (end 23.125045 19.399987) (width 0.2) (layer B.Cu) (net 12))
 (segment (start 22.150045 18.399987) (end 22.150045 18.424987) (width 0.2) (layer B.Cu) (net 12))
 (segment (start 21.175045 16.849987) (end 21.175045 18.399987) (width 0.2) (layer B.Cu) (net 11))
 (segment (start 21.175045 18.424987) (end 22.150045 19.399987) (width 0.2) (layer B.Cu) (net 11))
 (segment (start 21.175045 18.399987) (end 21.175045 18.424987) (width 0.2) (layer B.Cu) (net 11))
 (segment (start 21.825045 10.249987) (end 22.525045 9.549987) (width 0.2) (layer B.Cu) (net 4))
 (segment (start 21.825045 11.149987) (end 21.825045 10.249987) (width 0.2) (layer B.Cu) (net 4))
 (segment (start 21.175045 9.899987) (end 21.525045 9.549987) (width 0.2) (layer B.Cu) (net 5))
 (segment (start 21.175045 11.149987) (end 21.175045 9.899987) (width 0.2) (layer B.Cu) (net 5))
 (segment (start 21.525045 9.549987) (end 21.525045 8.449987) (width 0.2) (layer B.Cu) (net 5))
 (segment (start 20.525045 11.149987) (end 20.525045 9.549987) (width 0.2) (layer B.Cu) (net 6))
 (segment (start 17.875045 16.799987) (end 17.925045 16.849987) (width 0.2) (layer B.Cu) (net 8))
 (segment (start 16.925045 16.799987) (end 17.875045 16.799987) (width 0.2) (layer B.Cu) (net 8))
 (segment (start 18.575045 9.549987) (end 18.575045 11.149987) (width 0.2) (layer B.Cu) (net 7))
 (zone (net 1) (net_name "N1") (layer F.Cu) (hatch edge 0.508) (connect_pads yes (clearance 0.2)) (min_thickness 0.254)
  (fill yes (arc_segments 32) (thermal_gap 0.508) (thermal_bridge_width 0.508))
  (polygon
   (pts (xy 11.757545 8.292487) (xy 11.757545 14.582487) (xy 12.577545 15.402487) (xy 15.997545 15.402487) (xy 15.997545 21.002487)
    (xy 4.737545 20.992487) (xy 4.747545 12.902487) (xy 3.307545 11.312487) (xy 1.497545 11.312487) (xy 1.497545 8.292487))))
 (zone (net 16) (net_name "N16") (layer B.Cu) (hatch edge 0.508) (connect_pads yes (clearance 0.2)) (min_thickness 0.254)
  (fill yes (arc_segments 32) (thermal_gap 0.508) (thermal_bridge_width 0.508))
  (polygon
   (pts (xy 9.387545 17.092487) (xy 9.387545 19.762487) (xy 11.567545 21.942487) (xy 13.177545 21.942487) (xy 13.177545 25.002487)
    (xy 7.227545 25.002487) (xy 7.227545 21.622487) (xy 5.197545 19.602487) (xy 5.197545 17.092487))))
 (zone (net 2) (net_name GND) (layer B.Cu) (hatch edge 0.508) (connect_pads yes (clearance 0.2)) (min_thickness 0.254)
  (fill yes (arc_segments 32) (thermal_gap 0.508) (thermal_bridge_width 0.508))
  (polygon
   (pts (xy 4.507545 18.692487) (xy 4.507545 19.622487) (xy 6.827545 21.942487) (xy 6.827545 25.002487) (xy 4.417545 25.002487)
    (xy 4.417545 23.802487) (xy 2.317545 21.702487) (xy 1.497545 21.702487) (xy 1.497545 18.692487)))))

